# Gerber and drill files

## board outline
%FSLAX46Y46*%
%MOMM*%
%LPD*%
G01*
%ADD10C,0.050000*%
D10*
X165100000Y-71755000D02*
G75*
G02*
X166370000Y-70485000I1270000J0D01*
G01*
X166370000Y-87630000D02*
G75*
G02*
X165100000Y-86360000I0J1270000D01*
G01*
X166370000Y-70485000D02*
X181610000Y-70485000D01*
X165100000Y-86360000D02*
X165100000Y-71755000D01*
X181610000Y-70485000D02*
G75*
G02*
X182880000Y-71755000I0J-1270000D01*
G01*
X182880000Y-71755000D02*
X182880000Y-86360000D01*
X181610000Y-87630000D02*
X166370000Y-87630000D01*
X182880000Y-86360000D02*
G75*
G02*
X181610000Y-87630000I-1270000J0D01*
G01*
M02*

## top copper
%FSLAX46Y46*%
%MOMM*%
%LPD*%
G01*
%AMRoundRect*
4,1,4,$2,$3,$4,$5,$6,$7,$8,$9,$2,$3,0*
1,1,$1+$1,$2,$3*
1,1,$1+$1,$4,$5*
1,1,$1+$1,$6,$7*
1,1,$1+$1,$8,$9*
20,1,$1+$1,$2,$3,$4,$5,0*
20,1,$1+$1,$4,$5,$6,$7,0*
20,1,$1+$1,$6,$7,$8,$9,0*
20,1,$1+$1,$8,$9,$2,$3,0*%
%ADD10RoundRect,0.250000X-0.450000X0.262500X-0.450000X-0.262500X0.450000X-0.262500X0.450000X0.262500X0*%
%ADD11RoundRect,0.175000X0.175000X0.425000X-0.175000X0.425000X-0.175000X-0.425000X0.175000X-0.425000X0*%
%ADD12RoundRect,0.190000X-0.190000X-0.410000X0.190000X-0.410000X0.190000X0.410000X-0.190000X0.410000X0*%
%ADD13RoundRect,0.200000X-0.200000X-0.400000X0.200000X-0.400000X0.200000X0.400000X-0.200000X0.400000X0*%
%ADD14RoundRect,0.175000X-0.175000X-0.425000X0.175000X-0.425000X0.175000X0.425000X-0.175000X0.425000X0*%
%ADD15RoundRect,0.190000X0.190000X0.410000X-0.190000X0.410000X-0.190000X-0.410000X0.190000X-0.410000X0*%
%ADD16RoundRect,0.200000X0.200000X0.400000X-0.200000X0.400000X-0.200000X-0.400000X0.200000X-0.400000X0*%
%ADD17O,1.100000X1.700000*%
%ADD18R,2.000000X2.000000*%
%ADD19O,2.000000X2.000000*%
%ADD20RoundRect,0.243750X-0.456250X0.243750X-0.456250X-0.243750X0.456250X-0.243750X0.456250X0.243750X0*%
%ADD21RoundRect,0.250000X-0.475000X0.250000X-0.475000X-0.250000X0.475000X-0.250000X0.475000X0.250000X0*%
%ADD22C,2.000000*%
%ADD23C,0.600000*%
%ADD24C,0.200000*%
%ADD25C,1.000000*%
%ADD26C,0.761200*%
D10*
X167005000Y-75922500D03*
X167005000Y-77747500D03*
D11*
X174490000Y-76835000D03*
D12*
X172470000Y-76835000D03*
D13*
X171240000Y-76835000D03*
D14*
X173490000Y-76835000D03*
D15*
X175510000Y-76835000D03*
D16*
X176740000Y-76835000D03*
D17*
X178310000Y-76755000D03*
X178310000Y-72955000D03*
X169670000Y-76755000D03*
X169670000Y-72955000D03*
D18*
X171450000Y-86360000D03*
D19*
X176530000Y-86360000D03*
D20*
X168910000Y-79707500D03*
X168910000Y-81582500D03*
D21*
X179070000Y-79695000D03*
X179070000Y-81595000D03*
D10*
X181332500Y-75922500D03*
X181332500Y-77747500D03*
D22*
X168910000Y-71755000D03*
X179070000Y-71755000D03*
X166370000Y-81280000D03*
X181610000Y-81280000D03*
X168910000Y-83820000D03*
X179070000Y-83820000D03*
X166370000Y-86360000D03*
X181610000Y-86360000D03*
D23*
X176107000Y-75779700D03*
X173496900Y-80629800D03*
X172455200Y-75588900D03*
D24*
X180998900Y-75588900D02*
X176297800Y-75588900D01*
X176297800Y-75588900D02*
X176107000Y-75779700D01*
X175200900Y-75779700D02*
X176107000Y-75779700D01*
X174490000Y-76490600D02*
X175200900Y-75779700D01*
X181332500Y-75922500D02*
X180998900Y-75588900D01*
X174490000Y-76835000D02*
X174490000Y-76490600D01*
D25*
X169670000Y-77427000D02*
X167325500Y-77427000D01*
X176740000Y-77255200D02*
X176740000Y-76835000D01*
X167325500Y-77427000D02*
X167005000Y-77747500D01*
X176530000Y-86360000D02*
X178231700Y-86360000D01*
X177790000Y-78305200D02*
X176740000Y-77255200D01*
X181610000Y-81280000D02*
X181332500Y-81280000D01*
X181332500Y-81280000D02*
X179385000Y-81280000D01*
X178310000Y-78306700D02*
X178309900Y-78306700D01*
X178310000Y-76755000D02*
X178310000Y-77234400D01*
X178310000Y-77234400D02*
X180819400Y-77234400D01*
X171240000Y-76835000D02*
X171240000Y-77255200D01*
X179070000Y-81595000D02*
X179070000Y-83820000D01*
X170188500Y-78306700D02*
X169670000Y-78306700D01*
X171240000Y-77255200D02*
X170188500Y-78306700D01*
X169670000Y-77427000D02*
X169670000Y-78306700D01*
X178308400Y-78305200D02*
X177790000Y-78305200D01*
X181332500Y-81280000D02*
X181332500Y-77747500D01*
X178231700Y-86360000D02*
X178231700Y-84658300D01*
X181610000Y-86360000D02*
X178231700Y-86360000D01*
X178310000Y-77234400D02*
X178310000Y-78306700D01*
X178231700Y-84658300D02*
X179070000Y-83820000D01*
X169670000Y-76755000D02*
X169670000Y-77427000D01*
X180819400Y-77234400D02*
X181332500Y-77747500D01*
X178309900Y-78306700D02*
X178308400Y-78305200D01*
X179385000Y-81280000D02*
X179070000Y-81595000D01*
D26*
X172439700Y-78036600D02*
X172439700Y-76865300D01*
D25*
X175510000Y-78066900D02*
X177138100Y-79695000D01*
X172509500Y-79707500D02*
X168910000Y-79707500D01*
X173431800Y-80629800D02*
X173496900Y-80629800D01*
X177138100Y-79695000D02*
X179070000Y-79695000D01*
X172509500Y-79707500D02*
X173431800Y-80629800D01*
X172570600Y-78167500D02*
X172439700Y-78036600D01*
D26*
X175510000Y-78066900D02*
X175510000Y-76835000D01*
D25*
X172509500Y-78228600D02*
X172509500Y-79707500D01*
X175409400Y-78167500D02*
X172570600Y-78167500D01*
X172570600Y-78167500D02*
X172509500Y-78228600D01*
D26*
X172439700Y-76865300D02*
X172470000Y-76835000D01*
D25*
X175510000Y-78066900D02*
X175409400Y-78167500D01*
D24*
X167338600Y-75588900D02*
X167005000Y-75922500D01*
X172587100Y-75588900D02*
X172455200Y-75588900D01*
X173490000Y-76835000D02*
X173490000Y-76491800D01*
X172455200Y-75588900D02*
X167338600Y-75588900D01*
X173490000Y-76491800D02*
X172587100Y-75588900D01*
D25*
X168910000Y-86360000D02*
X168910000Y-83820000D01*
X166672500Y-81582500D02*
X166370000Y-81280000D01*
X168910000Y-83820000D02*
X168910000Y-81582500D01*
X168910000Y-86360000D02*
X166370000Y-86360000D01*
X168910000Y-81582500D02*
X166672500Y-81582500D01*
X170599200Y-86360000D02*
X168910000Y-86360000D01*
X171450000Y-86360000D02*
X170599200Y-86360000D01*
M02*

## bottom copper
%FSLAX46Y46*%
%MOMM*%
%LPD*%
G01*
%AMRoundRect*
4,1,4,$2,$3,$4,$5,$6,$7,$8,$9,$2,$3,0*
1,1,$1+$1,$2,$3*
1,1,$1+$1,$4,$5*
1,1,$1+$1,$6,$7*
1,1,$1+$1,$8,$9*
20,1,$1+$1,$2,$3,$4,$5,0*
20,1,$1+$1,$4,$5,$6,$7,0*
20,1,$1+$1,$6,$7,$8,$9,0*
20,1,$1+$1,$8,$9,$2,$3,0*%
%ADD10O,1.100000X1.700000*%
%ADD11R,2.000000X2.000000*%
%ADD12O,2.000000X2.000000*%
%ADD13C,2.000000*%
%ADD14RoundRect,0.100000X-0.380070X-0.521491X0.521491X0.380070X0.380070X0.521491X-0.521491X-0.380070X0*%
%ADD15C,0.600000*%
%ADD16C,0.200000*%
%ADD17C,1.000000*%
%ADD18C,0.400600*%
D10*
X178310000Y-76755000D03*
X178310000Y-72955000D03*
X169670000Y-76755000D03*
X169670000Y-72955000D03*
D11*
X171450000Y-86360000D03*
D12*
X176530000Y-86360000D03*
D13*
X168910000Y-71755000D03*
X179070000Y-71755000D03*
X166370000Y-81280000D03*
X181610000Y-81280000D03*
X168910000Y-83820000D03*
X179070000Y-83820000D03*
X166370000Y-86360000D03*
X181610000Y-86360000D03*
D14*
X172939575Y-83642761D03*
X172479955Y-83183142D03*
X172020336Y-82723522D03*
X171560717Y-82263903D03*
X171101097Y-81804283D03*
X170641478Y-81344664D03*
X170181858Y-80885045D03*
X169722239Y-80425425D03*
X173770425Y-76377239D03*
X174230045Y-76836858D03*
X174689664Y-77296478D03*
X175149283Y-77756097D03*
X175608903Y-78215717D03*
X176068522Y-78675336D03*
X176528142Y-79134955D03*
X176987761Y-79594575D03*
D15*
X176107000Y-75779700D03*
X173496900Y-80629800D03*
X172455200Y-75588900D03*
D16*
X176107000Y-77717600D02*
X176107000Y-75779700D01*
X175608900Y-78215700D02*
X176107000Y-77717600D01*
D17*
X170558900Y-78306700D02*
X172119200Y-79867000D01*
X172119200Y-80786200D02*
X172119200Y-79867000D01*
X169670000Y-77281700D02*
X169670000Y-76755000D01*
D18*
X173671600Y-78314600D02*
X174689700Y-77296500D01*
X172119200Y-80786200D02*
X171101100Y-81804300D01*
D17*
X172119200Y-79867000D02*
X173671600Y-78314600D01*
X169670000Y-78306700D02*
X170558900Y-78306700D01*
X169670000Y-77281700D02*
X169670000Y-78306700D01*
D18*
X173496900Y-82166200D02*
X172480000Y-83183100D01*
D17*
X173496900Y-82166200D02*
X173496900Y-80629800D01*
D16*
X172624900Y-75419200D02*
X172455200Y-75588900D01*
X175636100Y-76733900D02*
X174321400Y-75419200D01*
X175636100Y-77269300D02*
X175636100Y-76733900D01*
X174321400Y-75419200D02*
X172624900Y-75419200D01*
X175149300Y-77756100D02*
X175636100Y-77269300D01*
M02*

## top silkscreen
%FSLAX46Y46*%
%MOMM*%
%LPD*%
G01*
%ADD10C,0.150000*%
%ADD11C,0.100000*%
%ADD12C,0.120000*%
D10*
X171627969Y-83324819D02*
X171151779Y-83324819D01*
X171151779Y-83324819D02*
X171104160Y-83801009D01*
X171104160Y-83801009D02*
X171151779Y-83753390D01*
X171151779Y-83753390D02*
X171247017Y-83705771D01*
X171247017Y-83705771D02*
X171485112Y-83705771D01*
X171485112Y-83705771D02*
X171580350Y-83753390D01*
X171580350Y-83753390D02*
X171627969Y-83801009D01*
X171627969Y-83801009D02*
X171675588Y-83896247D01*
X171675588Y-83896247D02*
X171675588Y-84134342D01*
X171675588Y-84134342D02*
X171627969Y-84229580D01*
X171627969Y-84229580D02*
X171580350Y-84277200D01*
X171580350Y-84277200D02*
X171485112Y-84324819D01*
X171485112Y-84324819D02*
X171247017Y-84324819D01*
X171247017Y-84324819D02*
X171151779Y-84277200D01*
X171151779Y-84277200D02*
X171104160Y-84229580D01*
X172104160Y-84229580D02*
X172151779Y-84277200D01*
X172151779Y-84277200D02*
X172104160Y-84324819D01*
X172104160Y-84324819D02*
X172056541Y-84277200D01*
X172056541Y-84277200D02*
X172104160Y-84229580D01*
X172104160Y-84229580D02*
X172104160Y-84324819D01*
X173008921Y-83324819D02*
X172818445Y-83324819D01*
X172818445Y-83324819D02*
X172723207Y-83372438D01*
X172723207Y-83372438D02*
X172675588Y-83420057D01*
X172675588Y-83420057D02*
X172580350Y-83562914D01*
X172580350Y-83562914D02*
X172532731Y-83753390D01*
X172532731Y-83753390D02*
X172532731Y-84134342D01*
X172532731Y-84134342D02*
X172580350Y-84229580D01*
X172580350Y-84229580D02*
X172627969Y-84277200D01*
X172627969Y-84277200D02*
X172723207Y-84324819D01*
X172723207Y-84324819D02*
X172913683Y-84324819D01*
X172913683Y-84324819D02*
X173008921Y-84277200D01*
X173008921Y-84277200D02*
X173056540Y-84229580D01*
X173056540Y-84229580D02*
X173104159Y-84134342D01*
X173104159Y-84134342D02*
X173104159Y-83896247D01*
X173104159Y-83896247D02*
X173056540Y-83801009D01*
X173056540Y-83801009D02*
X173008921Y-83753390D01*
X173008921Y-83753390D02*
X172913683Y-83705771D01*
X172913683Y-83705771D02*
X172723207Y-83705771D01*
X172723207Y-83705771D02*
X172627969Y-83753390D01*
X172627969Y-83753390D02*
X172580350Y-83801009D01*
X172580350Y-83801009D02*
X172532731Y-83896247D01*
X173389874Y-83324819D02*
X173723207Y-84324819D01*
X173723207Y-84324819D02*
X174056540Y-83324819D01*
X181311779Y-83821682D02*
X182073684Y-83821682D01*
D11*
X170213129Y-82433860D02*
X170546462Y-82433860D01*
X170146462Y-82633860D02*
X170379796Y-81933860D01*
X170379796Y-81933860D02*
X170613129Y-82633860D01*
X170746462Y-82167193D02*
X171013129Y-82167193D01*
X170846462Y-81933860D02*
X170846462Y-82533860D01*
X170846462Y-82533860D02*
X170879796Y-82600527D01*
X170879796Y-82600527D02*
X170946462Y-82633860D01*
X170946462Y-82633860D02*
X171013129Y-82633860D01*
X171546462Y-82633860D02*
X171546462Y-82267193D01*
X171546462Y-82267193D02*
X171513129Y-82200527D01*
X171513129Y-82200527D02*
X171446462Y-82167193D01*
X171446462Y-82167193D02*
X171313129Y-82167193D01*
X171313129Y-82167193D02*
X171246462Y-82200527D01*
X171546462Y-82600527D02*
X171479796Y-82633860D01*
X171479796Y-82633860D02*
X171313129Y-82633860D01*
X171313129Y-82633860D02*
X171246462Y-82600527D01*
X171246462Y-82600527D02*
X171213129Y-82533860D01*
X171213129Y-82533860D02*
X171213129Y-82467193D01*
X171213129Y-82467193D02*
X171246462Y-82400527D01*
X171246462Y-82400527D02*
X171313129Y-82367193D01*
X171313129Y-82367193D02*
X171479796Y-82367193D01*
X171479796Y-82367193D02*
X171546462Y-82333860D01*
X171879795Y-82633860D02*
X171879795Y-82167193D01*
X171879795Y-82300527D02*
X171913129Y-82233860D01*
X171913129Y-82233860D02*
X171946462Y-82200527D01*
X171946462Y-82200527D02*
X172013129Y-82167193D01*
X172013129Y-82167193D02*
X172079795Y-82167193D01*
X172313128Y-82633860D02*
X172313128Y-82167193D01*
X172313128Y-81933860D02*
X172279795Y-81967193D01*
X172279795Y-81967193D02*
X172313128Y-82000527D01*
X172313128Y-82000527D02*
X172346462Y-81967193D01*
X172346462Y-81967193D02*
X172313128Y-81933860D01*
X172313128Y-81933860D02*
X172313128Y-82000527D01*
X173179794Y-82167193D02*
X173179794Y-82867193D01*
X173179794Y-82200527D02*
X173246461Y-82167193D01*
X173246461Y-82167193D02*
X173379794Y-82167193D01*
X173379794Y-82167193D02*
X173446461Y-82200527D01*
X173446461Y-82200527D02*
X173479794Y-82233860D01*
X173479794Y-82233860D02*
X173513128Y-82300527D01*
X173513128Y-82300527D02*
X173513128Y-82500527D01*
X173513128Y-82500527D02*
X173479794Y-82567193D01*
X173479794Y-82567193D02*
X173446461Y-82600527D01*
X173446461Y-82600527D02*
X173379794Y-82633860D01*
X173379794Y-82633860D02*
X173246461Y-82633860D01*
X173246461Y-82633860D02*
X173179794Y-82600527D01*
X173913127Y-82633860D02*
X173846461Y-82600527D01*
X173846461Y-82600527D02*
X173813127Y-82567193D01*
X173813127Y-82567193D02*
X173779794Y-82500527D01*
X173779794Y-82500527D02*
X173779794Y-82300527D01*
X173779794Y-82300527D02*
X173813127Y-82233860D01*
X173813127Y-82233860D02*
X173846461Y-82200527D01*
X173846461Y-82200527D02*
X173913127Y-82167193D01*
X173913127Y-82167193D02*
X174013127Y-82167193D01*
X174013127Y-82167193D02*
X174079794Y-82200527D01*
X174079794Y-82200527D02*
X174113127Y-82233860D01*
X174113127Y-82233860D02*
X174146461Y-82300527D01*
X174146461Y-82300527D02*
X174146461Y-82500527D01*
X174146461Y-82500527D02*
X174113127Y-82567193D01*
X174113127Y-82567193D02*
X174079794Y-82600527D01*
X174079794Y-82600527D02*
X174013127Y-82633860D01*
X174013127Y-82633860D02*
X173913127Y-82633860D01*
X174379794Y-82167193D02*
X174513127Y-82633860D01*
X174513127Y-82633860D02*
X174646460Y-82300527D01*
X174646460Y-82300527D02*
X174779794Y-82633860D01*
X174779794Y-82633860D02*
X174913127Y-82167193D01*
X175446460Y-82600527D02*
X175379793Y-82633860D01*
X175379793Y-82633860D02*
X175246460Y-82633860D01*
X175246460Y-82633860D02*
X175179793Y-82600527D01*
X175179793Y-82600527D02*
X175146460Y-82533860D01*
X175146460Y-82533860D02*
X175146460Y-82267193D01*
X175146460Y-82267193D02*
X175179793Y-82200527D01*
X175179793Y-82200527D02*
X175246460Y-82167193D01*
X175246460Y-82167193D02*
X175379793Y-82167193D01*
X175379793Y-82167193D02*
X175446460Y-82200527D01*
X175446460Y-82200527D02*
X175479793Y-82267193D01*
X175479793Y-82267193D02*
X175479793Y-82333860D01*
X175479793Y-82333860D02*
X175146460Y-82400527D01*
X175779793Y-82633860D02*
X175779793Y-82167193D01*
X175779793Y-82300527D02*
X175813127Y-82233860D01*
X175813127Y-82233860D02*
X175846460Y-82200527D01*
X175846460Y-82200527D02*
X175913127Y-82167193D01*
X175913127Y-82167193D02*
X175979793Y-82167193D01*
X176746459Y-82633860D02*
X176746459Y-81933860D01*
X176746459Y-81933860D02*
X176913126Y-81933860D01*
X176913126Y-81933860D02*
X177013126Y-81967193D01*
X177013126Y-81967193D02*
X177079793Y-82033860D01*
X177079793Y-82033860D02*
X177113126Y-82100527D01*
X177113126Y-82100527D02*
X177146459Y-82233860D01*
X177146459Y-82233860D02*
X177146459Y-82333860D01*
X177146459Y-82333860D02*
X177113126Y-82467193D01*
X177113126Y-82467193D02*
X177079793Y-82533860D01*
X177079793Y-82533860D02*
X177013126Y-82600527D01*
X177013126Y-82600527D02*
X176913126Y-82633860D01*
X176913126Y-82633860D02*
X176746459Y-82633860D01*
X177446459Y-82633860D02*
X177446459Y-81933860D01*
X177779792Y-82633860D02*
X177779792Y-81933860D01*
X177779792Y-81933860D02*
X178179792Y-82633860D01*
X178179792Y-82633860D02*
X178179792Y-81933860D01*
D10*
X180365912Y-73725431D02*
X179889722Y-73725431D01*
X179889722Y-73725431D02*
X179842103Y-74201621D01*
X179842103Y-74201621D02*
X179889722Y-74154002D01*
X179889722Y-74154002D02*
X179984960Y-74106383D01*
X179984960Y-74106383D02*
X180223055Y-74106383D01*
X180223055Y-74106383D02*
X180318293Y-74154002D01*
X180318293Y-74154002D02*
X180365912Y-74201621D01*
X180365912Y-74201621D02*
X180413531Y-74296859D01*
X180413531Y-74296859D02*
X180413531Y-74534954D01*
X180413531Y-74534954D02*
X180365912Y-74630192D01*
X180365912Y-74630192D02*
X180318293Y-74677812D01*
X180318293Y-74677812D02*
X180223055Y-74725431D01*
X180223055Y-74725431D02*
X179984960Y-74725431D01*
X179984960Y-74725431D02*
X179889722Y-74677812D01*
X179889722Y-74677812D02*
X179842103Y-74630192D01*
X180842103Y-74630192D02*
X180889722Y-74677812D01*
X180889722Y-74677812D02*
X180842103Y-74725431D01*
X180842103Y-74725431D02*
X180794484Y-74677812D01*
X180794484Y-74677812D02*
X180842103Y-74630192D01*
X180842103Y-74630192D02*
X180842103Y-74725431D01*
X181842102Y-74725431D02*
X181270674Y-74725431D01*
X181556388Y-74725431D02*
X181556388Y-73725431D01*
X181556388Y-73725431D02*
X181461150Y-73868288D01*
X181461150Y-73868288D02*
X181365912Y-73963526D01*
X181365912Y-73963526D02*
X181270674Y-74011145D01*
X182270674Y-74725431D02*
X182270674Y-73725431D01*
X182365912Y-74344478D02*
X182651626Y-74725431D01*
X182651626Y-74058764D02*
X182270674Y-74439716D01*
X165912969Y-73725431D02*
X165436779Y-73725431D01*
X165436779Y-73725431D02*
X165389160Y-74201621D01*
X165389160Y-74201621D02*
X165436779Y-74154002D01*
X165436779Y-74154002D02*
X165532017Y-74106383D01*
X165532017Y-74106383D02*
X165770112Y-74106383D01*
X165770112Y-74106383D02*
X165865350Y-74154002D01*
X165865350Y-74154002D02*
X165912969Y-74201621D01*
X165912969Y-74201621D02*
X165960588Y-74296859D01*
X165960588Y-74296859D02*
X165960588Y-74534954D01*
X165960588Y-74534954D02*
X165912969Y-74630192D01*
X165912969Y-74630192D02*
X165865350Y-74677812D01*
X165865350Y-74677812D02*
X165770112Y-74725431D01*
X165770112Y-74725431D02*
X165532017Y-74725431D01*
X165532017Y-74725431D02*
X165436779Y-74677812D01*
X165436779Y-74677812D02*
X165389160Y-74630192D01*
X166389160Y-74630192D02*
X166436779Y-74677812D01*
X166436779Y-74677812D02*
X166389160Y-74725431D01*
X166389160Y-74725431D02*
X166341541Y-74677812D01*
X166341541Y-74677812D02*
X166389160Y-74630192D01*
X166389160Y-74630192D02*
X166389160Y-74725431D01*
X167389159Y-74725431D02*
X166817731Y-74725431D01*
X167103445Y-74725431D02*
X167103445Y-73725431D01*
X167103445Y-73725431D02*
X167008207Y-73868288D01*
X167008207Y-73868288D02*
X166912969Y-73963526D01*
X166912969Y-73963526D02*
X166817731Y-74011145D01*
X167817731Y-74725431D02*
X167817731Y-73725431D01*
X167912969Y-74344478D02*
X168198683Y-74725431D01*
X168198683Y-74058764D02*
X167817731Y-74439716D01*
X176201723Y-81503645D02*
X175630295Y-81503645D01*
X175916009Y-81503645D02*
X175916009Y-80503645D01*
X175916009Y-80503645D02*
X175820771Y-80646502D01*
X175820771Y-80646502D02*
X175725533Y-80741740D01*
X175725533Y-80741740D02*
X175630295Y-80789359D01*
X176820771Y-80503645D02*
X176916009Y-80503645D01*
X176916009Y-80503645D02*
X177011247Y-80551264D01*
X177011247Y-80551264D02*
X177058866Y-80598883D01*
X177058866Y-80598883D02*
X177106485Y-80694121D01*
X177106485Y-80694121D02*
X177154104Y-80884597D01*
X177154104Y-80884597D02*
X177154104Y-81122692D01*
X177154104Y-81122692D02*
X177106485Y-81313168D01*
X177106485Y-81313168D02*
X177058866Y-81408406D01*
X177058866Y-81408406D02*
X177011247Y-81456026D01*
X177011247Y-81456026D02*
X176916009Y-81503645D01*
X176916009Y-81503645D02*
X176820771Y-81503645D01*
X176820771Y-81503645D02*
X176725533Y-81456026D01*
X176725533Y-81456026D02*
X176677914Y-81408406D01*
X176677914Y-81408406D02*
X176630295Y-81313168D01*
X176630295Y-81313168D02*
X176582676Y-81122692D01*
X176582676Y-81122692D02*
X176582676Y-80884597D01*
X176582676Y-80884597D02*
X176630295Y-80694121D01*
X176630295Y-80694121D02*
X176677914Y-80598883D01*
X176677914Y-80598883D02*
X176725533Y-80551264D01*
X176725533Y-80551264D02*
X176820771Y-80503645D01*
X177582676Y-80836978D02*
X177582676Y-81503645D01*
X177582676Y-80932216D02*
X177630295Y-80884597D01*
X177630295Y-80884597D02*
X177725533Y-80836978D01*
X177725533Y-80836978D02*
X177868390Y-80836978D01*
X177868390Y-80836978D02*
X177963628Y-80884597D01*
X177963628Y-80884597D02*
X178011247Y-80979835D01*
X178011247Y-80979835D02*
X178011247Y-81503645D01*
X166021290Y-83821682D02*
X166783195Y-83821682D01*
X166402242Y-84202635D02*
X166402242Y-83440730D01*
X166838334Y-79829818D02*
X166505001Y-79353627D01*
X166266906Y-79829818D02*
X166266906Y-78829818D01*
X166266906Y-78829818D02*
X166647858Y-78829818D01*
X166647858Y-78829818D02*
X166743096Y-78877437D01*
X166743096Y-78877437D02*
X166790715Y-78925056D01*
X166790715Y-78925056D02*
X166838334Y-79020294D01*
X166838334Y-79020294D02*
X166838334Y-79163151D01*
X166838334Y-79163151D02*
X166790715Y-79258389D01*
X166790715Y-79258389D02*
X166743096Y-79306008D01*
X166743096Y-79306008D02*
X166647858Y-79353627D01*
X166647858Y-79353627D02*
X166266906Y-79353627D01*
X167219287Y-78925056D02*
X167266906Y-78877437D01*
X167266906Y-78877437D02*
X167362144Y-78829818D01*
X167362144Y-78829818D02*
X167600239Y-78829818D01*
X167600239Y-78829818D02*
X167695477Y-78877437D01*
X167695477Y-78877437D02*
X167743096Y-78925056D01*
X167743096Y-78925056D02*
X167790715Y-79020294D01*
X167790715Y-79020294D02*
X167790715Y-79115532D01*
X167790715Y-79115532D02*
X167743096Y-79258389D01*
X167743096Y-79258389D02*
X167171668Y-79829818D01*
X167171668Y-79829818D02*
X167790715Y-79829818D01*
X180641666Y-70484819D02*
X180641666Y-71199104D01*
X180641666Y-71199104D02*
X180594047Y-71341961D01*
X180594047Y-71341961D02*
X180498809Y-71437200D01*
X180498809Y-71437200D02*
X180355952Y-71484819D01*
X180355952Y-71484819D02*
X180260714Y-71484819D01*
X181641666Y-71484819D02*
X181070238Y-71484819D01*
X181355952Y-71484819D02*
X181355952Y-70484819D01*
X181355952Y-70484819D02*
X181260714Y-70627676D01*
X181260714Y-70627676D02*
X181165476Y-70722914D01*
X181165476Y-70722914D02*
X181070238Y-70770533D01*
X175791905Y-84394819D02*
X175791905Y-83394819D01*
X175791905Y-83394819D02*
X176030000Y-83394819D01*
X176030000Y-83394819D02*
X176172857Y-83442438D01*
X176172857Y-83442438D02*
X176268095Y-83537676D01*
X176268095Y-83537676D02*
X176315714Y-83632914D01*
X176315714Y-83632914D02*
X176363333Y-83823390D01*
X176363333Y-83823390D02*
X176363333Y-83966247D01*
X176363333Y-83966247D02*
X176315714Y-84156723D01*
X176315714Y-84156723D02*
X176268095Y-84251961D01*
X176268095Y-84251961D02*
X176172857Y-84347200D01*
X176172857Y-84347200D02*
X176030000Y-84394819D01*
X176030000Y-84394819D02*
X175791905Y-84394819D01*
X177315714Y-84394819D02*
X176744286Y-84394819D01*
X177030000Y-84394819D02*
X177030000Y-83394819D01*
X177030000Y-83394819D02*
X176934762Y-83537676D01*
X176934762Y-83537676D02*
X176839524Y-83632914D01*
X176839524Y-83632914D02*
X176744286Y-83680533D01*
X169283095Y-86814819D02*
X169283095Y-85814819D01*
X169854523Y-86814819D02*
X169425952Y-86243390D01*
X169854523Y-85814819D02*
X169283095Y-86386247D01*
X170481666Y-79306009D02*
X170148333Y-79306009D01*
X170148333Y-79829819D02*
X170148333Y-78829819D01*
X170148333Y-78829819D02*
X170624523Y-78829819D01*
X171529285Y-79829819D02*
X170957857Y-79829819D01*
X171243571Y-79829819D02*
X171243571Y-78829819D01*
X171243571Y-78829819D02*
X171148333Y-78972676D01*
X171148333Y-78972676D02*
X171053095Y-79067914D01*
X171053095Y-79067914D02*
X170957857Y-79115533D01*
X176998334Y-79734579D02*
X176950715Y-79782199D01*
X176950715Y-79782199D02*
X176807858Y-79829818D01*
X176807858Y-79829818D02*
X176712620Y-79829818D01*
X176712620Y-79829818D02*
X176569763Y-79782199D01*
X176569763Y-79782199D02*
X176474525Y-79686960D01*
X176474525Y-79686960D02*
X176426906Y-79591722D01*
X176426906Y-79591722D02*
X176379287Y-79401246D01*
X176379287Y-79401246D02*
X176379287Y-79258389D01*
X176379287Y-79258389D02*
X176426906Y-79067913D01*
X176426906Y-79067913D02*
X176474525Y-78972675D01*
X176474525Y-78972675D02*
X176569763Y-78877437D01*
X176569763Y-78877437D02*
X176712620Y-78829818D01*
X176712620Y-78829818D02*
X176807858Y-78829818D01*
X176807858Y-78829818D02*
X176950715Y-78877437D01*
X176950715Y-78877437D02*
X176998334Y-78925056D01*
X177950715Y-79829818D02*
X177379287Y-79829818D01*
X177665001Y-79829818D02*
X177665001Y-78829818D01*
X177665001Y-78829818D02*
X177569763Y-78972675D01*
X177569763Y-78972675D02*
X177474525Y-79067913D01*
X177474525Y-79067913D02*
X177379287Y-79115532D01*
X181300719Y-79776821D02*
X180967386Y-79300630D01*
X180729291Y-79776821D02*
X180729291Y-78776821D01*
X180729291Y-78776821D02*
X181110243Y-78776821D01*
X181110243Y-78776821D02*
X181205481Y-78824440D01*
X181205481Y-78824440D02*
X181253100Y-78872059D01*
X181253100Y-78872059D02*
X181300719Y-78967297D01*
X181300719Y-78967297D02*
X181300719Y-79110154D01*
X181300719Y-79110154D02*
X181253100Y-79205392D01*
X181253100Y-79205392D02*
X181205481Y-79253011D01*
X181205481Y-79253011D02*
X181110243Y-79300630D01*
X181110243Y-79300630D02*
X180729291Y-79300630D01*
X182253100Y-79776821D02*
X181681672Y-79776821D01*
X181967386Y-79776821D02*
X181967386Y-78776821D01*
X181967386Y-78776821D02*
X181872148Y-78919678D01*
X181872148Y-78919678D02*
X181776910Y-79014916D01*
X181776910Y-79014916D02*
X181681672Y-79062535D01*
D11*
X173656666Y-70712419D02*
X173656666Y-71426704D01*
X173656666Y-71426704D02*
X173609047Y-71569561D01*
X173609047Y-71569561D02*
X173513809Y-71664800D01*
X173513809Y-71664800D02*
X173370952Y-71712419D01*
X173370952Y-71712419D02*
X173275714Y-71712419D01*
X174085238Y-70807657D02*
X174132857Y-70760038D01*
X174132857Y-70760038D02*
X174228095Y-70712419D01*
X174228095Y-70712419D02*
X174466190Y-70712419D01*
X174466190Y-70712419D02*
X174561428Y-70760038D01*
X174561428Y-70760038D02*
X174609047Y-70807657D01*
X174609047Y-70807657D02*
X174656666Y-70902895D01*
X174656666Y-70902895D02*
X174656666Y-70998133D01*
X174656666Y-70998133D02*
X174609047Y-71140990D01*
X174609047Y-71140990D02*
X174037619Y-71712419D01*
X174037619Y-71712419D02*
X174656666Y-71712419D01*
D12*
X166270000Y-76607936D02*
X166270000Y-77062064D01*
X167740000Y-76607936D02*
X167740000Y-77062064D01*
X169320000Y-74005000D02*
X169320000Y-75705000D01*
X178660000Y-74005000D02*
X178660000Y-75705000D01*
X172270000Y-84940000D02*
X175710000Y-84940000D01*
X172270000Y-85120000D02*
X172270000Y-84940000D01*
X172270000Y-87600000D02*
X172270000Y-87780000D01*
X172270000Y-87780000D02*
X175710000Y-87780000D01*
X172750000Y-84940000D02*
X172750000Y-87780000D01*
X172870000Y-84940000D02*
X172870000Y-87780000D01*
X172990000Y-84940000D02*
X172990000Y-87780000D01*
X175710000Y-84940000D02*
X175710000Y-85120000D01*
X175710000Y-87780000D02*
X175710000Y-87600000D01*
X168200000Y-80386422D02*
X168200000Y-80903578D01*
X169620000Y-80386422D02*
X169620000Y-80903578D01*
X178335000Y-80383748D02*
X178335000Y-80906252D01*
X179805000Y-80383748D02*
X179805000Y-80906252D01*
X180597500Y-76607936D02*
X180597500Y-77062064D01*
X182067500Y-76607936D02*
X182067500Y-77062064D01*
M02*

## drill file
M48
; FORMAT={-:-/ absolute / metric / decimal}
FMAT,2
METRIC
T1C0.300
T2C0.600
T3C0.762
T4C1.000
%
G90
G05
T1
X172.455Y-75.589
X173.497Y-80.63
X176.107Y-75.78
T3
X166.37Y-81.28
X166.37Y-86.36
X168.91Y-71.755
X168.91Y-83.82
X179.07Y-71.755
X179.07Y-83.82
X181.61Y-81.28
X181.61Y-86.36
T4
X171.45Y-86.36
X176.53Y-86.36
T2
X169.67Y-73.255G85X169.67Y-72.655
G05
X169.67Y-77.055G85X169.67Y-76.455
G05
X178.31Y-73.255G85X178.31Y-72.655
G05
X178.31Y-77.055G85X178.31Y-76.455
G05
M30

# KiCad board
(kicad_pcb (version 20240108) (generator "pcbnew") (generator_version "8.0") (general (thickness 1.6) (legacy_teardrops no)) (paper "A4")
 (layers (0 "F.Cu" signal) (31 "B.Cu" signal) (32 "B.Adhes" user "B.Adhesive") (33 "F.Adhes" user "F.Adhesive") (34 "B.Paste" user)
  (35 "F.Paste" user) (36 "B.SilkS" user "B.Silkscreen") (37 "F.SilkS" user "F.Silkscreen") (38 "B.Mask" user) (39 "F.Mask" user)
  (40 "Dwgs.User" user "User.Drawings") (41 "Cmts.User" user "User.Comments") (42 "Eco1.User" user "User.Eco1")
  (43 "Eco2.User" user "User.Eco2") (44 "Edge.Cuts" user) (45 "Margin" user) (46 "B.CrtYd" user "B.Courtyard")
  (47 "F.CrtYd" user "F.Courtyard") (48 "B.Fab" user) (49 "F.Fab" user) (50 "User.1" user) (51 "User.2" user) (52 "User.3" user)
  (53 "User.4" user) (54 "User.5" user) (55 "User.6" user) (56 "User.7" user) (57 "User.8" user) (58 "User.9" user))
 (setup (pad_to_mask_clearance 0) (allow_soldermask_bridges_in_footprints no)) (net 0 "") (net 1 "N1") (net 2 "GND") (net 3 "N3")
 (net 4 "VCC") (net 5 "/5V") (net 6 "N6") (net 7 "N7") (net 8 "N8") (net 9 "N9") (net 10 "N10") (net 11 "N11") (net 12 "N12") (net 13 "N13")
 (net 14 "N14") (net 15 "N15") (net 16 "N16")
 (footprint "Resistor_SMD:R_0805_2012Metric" (layer "F.Cu") (at 167.005 76.835 -90)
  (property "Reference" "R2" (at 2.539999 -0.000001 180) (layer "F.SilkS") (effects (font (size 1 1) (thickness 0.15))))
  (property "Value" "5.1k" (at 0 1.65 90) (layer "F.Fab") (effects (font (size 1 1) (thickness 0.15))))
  (fp_line (start -0.227064 0.735) (end 0.227064 0.735) (stroke (width 0.12) (type solid)) (layer "F.SilkS"))
  (fp_line (start -0.227064 -0.735) (end 0.227064 -0.735) (stroke (width 0.12) (type solid)) (layer "F.SilkS"))
  (pad "1" smd roundrect (at -0.9125 0 270) (size 1.025 1.4) (layers "F.Cu" "F.Paste" "F.Mask") (roundrect_rratio 0.243902439) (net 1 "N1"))
  (pad "2" smd roundrect (at 0.9125 0 270) (size 1.025 1.4) (layers "F.Cu" "F.Paste" "F.Mask") (roundrect_rratio 0.243902439) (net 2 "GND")))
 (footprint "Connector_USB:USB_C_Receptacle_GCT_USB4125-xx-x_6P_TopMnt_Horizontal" (layer "F.Cu") (at 173.99 73.755 180)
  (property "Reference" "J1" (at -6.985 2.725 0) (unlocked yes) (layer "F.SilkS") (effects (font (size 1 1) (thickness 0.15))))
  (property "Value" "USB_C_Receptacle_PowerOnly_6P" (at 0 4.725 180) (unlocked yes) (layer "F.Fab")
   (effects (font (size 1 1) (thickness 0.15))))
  (fp_line (start 4.67 -0.25) (end 4.67 -1.95) (stroke (width 0.12) (type solid)) (layer "F.SilkS"))
  (fp_line (start -4.67 -0.25) (end -4.67 -1.95) (stroke (width 0.12) (type solid)) (layer "F.SilkS"))
  (pad "A5" smd roundrect (at -0.5 -3.08 180) (size 0.7 1.2) (layers "F.Cu" "F.Paste" "F.Mask") (roundrect_rratio 0.25) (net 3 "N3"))
  (pad "A9" smd roundrect (at 1.52 -3.08) (size 0.76 1.2) (layers "F.Cu" "F.Paste" "F.Mask") (roundrect_rratio 0.25) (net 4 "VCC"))
  (pad "A12" smd roundrect (at 2.75 -3.08) (size 0.8 1.2) (layers "F.Cu" "F.Paste" "F.Mask") (roundrect_rratio 0.25) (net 2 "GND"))
  (pad "B5" smd roundrect (at 0.5 -3.08) (size 0.7 1.2) (layers "F.Cu" "F.Paste" "F.Mask") (roundrect_rratio 0.25) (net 1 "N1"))
  (pad "B9" smd roundrect (at -1.52 -3.08 180) (size 0.76 1.2) (layers "F.Cu" "F.Paste" "F.Mask") (roundrect_rratio 0.25) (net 4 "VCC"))
  (pad "B12" smd roundrect (at -2.75 -3.08 180) (size 0.8 1.2) (layers "F.Cu" "F.Paste" "F.Mask") (roundrect_rratio 0.25) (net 2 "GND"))
  (pad "S1" thru_hole oval (at -4.32 -3 180) (size 1.1 1.7) (drill oval 0.6 1.2) (layers "*.Cu" "*.Mask" "F.Paste")
   (remove_unused_layers no) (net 2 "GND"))
  (pad "S1" thru_hole oval (at -4.32 0.8 180) (size 1.1 1.7) (drill oval 0.6 1.2) (layers "*.Cu" "*.Mask" "F.Paste")
   (remove_unused_layers no) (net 2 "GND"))
  (pad "S1" thru_hole oval (at 4.32 -3 180) (size 1.1 1.7) (drill oval 0.6 1.2) (layers "*.Cu" "*.Mask" "F.Paste") (remove_unused_layers no)
   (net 2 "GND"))
  (pad "S1" thru_hole oval (at 4.32 0.8 180) (size 1.1 1.7) (drill oval 0.6 1.2) (layers "*.Cu" "*.Mask" "F.Paste")
   (remove_unused_layers no) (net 2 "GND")))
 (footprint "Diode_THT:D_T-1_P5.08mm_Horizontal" (layer "F.Cu") (at 171.45 86.36)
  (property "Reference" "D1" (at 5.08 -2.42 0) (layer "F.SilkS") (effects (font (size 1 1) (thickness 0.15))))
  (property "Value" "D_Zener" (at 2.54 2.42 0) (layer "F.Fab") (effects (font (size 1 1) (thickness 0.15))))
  (fp_line (start 0.82 -1.42) (end 4.26 -1.42) (stroke (width 0.12) (type solid)) (layer "F.SilkS"))
  (fp_line (start 0.82 -1.24) (end 0.82 -1.42) (stroke (width 0.12) (type solid)) (layer "F.SilkS"))
  (fp_line (start 0.82 1.24) (end 0.82 1.42) (stroke (width 0.12) (type solid)) (layer "F.SilkS"))
  (fp_line (start 0.82 1.42) (end 4.26 1.42) (stroke (width 0.12) (type solid)) (layer "F.SilkS"))
  (fp_line (start 1.3 -1.42) (end 1.3 1.42) (stroke (width 0.12) (type solid)) (layer "F.SilkS"))
  (fp_line (start 1.42 -1.42) (end 1.42 1.42) (stroke (width 0.12) (type solid)) (layer "F.SilkS"))
  (fp_line (start 1.54 -1.42) (end 1.54 1.42) (stroke (width 0.12) (type solid)) (layer "F.SilkS"))
  (fp_line (start 4.26 -1.42) (end 4.26 -1.24) (stroke (width 0.12) (type solid)) (layer "F.SilkS"))
  (fp_line (start 4.26 1.42) (end 4.26 1.24) (stroke (width 0.12) (type solid)) (layer "F.SilkS"))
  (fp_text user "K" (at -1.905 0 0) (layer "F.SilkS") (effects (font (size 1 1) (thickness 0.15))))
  (pad "1" thru_hole rect (at 0 0) (size 2 2) (drill 1) (layers "*.Cu" "*.Mask") (remove_unused_layers no) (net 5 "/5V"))
  (pad "2" thru_hole oval (at 5.08 0) (size 2 2) (drill 1) (layers "*.Cu" "*.Mask") (remove_unused_layers no) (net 2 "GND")))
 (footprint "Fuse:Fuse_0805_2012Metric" (layer "F.Cu") (at 168.91 80.645 -90)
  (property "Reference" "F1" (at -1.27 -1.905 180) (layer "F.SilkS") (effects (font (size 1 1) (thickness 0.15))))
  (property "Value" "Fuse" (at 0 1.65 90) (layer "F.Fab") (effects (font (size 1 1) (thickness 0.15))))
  (fp_line (start -0.258578 0.71) (end 0.258578 0.71) (stroke (width 0.12) (type solid)) (layer "F.SilkS"))
  (fp_line (start -0.258578 -0.71) (end 0.258578 -0.71) (stroke (width 0.12) (type solid)) (layer "F.SilkS"))
  (pad "1" smd roundrect (at -0.9375 0 270) (size 0.975 1.4) (layers "F.Cu" "F.Paste" "F.Mask") (roundrect_rratio 0.25) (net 4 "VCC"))
  (pad "2" smd roundrect (at 0.9375 0 270) (size 0.975 1.4) (layers "F.Cu" "F.Paste" "F.Mask") (roundrect_rratio 0.25) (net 5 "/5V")))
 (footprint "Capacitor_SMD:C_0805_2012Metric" (layer "F.Cu") (at 179.07 80.645 -90)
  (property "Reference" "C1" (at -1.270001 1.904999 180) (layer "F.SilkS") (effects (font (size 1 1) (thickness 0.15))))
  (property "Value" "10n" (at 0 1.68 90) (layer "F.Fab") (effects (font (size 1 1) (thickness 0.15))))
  (fp_line (start -0.261252 0.735) (end 0.261252 0.735) (stroke (width 0.12) (type solid)) (layer "F.SilkS"))
  (fp_line (start -0.261252 -0.735) (end 0.261252 -0.735) (stroke (width 0.12) (type solid)) (layer "F.SilkS"))
  (pad "1" smd roundrect (at -0.95 0 270) (size 1 1.45) (layers "F.Cu" "F.Paste" "F.Mask") (roundrect_rratio 0.25) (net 4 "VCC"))
  (pad "2" smd roundrect (at 0.95 0 270) (size 1 1.45) (layers "F.Cu" "F.Paste" "F.Mask") (roundrect_rratio 0.25) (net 2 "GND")))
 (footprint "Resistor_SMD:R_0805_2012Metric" (layer "F.Cu") (at 181.3325 76.835 -90)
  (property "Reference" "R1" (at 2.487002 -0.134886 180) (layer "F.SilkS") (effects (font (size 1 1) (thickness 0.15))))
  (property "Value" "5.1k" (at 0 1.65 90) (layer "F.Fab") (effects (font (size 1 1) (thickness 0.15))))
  (fp_line (start -0.227064 0.735) (end 0.227064 0.735) (stroke (width 0.12) (type solid)) (layer "F.SilkS"))
  (fp_line (start -0.227064 -0.735) (end 0.227064 -0.735) (stroke (width 0.12) (type solid)) (layer "F.SilkS"))
  (pad "1" smd roundrect (at -0.9125 0 270) (size 1.025 1.4) (layers "F.Cu" "F.Paste" "F.Mask") (roundrect_rratio 0.243902439) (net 3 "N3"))
  (pad "2" smd roundrect (at 0.9125 0 270) (size 1.025 1.4) (layers "F.Cu" "F.Paste" "F.Mask") (roundrect_rratio 0.243902439) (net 2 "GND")))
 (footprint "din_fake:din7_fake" (layer "F.Cu") (at 173.99 71.755)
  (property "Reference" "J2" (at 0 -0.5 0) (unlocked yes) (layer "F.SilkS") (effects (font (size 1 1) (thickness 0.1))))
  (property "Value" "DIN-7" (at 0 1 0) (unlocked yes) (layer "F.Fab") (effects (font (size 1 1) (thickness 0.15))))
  (pad "0" thru_hole circle (at -5.08 0) (size 2 2) (drill 0.762) (layers "*.Cu" "*.Mask") (remove_unused_layers no))
  (pad "0" thru_hole circle (at 5.08 0) (size 2 2) (drill 0.762) (layers "*.Cu" "*.Mask") (remove_unused_layers no))
  (pad "1" thru_hole circle (at -7.62 9.525) (size 2 2) (drill 0.762) (layers "*.Cu" "*.Mask") (remove_unused_layers no) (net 5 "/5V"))
  (pad "3" thru_hole circle (at 7.62 9.525) (size 2 2) (drill 0.762) (layers "*.Cu" "*.Mask") (remove_unused_layers no) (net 2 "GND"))
  (pad "4" thru_hole circle (at -5.08 12.065) (size 2 2) (drill 0.762) (layers "*.Cu" "*.Mask") (remove_unused_layers no) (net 5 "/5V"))
  (pad "5" thru_hole circle (at 5.08 12.065) (size 2 2) (drill 0.762) (layers "*.Cu" "*.Mask") (remove_unused_layers no) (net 2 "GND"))
  (pad "6" thru_hole circle (at -7.62 14.605) (size 2 2) (drill 0.762) (layers "*.Cu" "*.Mask") (remove_unused_layers no) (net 5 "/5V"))
  (pad "7" thru_hole circle (at 7.62 14.605) (size 2 2) (drill 0.762) (layers "*.Cu" "*.Mask") (remove_unused_layers no) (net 2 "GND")))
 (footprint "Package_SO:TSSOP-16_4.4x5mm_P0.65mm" (layer "B.Cu") (at 173.355 80.01 45)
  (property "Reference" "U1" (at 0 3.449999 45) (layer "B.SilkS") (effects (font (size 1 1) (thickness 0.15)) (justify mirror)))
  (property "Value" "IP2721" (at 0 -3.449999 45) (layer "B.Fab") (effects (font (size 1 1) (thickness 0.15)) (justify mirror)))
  (pad "1" smd roundrect (at -2.8625 2.275 45) (size 1.475 0.4) (layers "B.Cu" "B.Paste" "B.Mask") (roundrect_rratio 0.25) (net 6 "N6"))
  (pad "2" smd roundrect (at -2.8625 1.625 45) (size 1.475 0.4) (layers "B.Cu" "B.Paste" "B.Mask") (roundrect_rratio 0.25) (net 4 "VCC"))
  (pad "3" smd roundrect (at -2.8625 0.975 45) (size 1.475 0.4) (layers "B.Cu" "B.Paste" "B.Mask") (roundrect_rratio 0.25) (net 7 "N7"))
  (pad "4" smd roundrect (at -2.8625 0.325 45) (size 1.475 0.4) (layers "B.Cu" "B.Paste" "B.Mask") (roundrect_rratio 0.25) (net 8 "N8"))
  (pad "5" smd roundrect (at -2.8625 -0.325 45) (size 1.475 0.4) (layers "B.Cu" "B.Paste" "B.Mask") (roundrect_rratio 0.25) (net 2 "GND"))
  (pad "6" smd roundrect (at -2.8625 -0.975 45) (size 1.475 0.4) (layers "B.Cu" "B.Paste" "B.Mask") (roundrect_rratio 0.25) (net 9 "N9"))
  (pad "7" smd roundrect (at -2.8625 -1.625 45) (size 1.475 0.4) (layers "B.Cu" "B.Paste" "B.Mask") (roundrect_rratio 0.25) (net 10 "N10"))
  (pad "8" smd roundrect (at -2.8625 -2.275 45) (size 1.475 0.4) (layers "B.Cu" "B.Paste" "B.Mask") (roundrect_rratio 0.25) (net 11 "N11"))
  (pad "9" smd roundrect (at 2.8625 -2.275 45) (size 1.475 0.4) (layers "B.Cu" "B.Paste" "B.Mask") (roundrect_rratio 0.25) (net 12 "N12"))
  (pad "10" smd roundrect (at 2.8625 -1.625 45) (size 1.475 0.4) (layers "B.Cu" "B.Paste" "B.Mask") (roundrect_rratio 0.25) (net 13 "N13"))
  (pad "11" smd roundrect (at 2.8625 -0.975 45) (size 1.475 0.4) (layers "B.Cu" "B.Paste" "B.Mask") (roundrect_rratio 0.25) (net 2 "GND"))
  (pad "12" smd roundrect (at 2.8625 -0.325 45) (size 1.475 0.4) (layers "B.Cu" "B.Paste" "B.Mask") (roundrect_rratio 0.25) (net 1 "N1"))
  (pad "13" smd roundrect (at 2.8625 0.325 45) (size 1.475 0.4) (layers "B.Cu" "B.Paste" "B.Mask") (roundrect_rratio 0.25) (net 3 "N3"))
  (pad "14" smd roundrect (at 2.8625 0.975 45) (size 1.475 0.4) (layers "B.Cu" "B.Paste" "B.Mask") (roundrect_rratio 0.25) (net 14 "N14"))
  (pad "15" smd roundrect (at 2.8625 1.625 45) (size 1.475 0.4) (layers "B.Cu" "B.Paste" "B.Mask") (roundrect_rratio 0.25) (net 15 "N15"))
  (pad "16" smd roundrect (at 2.8625 2.275 45) (size 1.475 0.4) (layers "B.Cu" "B.Paste" "B.Mask") (roundrect_rratio 0.25) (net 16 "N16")))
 (gr_arc (start 165.1 71.755) (mid 165.471974 70.856974) (end 166.37 70.485) (stroke (width 0.05) (type default)) (layer "Edge.Cuts"))
 (gr_arc (start 166.37 87.63) (mid 165.471974 87.258026) (end 165.1 86.36) (stroke (width 0.05) (type default)) (layer "Edge.Cuts"))
 (gr_line (start 166.37 70.485) (end 181.61 70.485) (stroke (width 0.05) (type default)) (layer "Edge.Cuts"))
 (gr_line (start 165.1 86.36) (end 165.1 71.755) (stroke (width 0.05) (type default)) (layer "Edge.Cuts"))
 (gr_arc (start 181.61 70.485) (mid 182.508026 70.856974) (end 182.88 71.755) (stroke (width 0.05) (type default)) (layer "Edge.Cuts"))
 (gr_line (start 182.88 71.755) (end 182.88 86.36) (stroke (width 0.05) (type default)) (layer "Edge.Cuts"))
 (gr_line (start 181.61 87.63) (end 166.37 87.63) (stroke (width 0.05) (type default)) (layer "Edge.Cuts"))
 (gr_arc (start 182.88 86.36) (mid 182.508026 87.258026) (end 181.61 87.63) (stroke (width 0.05) (type default)) (layer "Edge.Cuts"))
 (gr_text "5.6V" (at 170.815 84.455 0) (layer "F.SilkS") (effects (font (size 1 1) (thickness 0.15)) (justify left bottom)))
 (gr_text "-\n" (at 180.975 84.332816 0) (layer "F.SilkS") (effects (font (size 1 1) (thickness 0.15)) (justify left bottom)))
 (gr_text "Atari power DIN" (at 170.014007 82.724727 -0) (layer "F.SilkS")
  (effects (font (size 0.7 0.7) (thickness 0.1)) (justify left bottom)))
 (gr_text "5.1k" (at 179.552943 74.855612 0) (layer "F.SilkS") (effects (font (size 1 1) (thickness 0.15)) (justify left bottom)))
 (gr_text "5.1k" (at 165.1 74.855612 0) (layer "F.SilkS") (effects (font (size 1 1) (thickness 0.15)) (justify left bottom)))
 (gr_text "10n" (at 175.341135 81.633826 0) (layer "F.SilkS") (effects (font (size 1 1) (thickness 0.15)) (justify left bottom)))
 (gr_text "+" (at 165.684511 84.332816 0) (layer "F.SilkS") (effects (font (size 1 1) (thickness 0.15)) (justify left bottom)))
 (segment (start 180.9989 75.5889) (end 176.2978 75.5889) (width 0.2) (layer "F.Cu") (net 3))
 (segment (start 176.2978 75.5889) (end 176.107 75.7797) (width 0.2) (layer "F.Cu") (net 3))
 (segment (start 175.2009 75.7797) (end 176.107 75.7797) (width 0.2) (layer "F.Cu") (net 3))
 (segment (start 174.49 76.4906) (end 175.2009 75.7797) (width 0.2) (layer "F.Cu") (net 3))
 (segment (start 181.3325 75.9225) (end 180.9989 75.5889) (width 0.2) (layer "F.Cu") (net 3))
 (segment (start 174.49 76.835) (end 174.49 76.4906) (width 0.2) (layer "F.Cu") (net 3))
 (via (at 176.107 75.7797) (size 0.6) (drill 0.3) (layers "F.Cu" "B.Cu") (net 3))
 (segment (start 176.107 77.7176) (end 176.107 75.7797) (width 0.2) (layer "B.Cu") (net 3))
 (segment (start 175.6089 78.2157) (end 176.107 77.7176) (width 0.2) (layer "B.Cu") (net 3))
 (segment (start 169.67 77.427) (end 167.3255 77.427) (width 1) (layer "F.Cu") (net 2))
 (segment (start 176.74 77.2552) (end 176.74 76.835) (width 1) (layer "F.Cu") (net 2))
 (segment (start 167.3255 77.427) (end 167.005 77.7475) (width 1) (layer "F.Cu") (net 2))
 (segment (start 176.53 86.36) (end 178.2317 86.36) (width 1) (layer "F.Cu") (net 2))
 (segment (start 177.79 78.3052) (end 176.74 77.2552) (width 1) (layer "F.Cu") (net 2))
 (segment (start 181.61 81.28) (end 181.3325 81.28) (width 1) (layer "F.Cu") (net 2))
 (segment (start 181.3325 81.28) (end 179.385 81.28) (width 1) (layer "F.Cu") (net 2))
 (segment (start 178.31 78.3067) (end 178.3099 78.3067) (width 1) (layer "F.Cu") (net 2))
 (segment (start 178.31 76.755) (end 178.31 77.2344) (width 1) (layer "F.Cu") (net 2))
 (segment (start 178.31 77.2344) (end 180.8194 77.2344) (width 1) (layer "F.Cu") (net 2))
 (segment (start 171.24 76.835) (end 171.24 77.2552) (width 1) (layer "F.Cu") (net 2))
 (segment (start 179.07 81.595) (end 179.07 83.82) (width 1) (layer "F.Cu") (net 2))
 (segment (start 170.1885 78.3067) (end 169.67 78.3067) (width 1) (layer "F.Cu") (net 2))
 (segment (start 171.24 77.2552) (end 170.1885 78.3067) (width 1) (layer "F.Cu") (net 2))
 (segment (start 169.67 77.427) (end 169.67 78.3067) (width 1) (layer "F.Cu") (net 2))
 (segment (start 178.3084 78.3052) (end 177.79 78.3052) (width 1) (layer "F.Cu") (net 2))
 (segment (start 181.3325 81.28) (end 181.3325 77.7475) (width 1) (layer "F.Cu") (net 2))
 (segment (start 178.2317 86.36) (end 178.2317 84.6583) (width 1) (layer "F.Cu") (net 2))
 (segment (start 181.61 86.36) (end 178.2317 86.36) (width 1) (layer "F.Cu") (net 2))
 (segment (start 178.31 77.2344) (end 178.31 78.3067) (width 1) (layer "F.Cu") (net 2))
 (segment (start 178.2317 84.6583) (end 179.07 83.82) (width 1) (layer "F.Cu") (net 2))
 (segment (start 169.67 76.755) (end 169.67 77.427) (width 1) (layer "F.Cu") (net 2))
 (segment (start 180.8194 77.2344) (end 181.3325 77.7475) (width 1) (layer "F.Cu") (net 2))
 (segment (start 178.3099 78.3067) (end 178.3084 78.3052) (width 1) (layer "F.Cu") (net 2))
 (segment (start 179.385 81.28) (end 179.07 81.595) (width 1) (layer "F.Cu") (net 2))
 (segment (start 170.5589 78.3067) (end 172.1192 79.867) (width 1) (layer "B.Cu") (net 2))
 (segment (start 172.1192 80.7862) (end 172.1192 79.867) (width 1) (layer "B.Cu") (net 2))
 (segment (start 169.67 77.2817) (end 169.67 76.755) (width 1) (layer "B.Cu") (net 2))
 (segment (start 173.6716 78.3146) (end 174.6897 77.2965) (width 0.4006) (layer "B.Cu") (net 2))
 (segment (start 172.1192 80.7862) (end 171.1011 81.8043) (width 0.4006) (layer "B.Cu") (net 2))
 (segment (start 172.1192 79.867) (end 173.6716 78.3146) (width 1) (layer "B.Cu") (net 2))
 (segment (start 169.67 78.3067) (end 170.5589 78.3067) (width 1) (layer "B.Cu") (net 2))
 (segment (start 169.67 77.2817) (end 169.67 78.3067) (width 1) (layer "B.Cu") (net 2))
 (segment (start 172.4397 78.0366) (end 172.4397 76.8653) (width 0.7612) (layer "F.Cu") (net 4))
 (segment (start 175.51 78.0669) (end 177.1381 79.695) (width 1) (layer "F.Cu") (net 4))
 (segment (start 172.5095 79.7075) (end 168.91 79.7075) (width 1) (layer "F.Cu") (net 4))
 (segment (start 173.4318 80.6298) (end 173.4969 80.6298) (width 1) (layer "F.Cu") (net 4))
 (segment (start 177.1381 79.695) (end 179.07 79.695) (width 1) (layer "F.Cu") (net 4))
 (segment (start 172.5095 79.7075) (end 173.4318 80.6298) (width 1) (layer "F.Cu") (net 4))
 (segment (start 172.5706 78.1675) (end 172.4397 78.0366) (width 1) (layer "F.Cu") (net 4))
 (segment (start 175.51 78.0669) (end 175.51 76.835) (width 0.7612) (layer "F.Cu") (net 4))
 (segment (start 172.5095 78.2286) (end 172.5095 79.7075) (width 1) (layer "F.Cu") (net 4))
 (segment (start 175.4094 78.1675) (end 172.5706 78.1675) (width 1) (layer "F.Cu") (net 4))
 (segment (start 172.5706 78.1675) (end 172.5095 78.2286) (width 1) (layer "F.Cu") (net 4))
 (segment (start 172.4397 76.8653) (end 172.47 76.835) (width 0.7612) (layer "F.Cu") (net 4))
 (segment (start 175.51 78.0669) (end 175.4094 78.1675) (width 1) (layer "F.Cu") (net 4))
 (via (at 173.4969 80.6298) (size 0.6) (drill 0.3) (layers "F.Cu" "B.Cu") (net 4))
 (segment (start 173.4969 82.1662) (end 172.48 83.1831) (width 0.4006) (layer "B.Cu") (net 4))
 (segment (start 173.4969 82.1662) (end 173.4969 80.6298) (width 1) (layer "B.Cu") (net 4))
 (segment (start 167.3386 75.5889) (end 167.005 75.9225) (width 0.2) (layer "F.Cu") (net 1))
 (segment (start 172.5871 75.5889) (end 172.4552 75.5889) (width 0.2) (layer "F.Cu") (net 1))
 (segment (start 173.49 76.835) (end 173.49 76.4918) (width 0.2) (layer "F.Cu") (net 1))
 (segment (start 172.4552 75.5889) (end 167.3386 75.5889) (width 0.2) (layer "F.Cu") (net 1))
 (segment (start 173.49 76.4918) (end 172.5871 75.5889) (width 0.2) (layer "F.Cu") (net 1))
 (via (at 172.4552 75.5889) (size 0.6) (drill 0.3) (layers "F.Cu" "B.Cu") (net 1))
 (segment (start 172.6249 75.4192) (end 172.4552 75.5889) (width 0.2) (layer "B.Cu") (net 1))
 (segment (start 175.6361 76.7339) (end 174.3214 75.4192) (width 0.2) (layer "B.Cu") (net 1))
 (segment (start 175.6361 77.2693) (end 175.6361 76.7339) (width 0.2) (layer "B.Cu") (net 1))
 (segment (start 174.3214 75.4192) (end 172.6249 75.4192) (width 0.2) (layer "B.Cu") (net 1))
 (segment (start 175.1493 77.7561) (end 175.6361 77.2693) (width 0.2) (layer "B.Cu") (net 1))
 (segment (start 168.91 86.36) (end 168.91 83.82) (width 1) (layer "F.Cu") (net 5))
 (segment (start 166.6725 81.5825) (end 166.37 81.28) (width 1) (layer "F.Cu") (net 5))
 (segment (start 168.91 83.82) (end 168.91 81.5825) (width 1) (layer "F.Cu") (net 5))
 (segment (start 168.91 86.36) (end 166.37 86.36) (width 1) (layer "F.Cu") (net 5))
 (segment (start 168.91 81.5825) (end 166.6725 81.5825) (width 1) (layer "F.Cu") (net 5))
 (segment (start 170.5992 86.36) (end 168.91 86.36) (width 1) (layer "F.Cu") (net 5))
 (segment (start 171.45 86.36) (end 170.5992 86.36) (width 1) (layer "F.Cu") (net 5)))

